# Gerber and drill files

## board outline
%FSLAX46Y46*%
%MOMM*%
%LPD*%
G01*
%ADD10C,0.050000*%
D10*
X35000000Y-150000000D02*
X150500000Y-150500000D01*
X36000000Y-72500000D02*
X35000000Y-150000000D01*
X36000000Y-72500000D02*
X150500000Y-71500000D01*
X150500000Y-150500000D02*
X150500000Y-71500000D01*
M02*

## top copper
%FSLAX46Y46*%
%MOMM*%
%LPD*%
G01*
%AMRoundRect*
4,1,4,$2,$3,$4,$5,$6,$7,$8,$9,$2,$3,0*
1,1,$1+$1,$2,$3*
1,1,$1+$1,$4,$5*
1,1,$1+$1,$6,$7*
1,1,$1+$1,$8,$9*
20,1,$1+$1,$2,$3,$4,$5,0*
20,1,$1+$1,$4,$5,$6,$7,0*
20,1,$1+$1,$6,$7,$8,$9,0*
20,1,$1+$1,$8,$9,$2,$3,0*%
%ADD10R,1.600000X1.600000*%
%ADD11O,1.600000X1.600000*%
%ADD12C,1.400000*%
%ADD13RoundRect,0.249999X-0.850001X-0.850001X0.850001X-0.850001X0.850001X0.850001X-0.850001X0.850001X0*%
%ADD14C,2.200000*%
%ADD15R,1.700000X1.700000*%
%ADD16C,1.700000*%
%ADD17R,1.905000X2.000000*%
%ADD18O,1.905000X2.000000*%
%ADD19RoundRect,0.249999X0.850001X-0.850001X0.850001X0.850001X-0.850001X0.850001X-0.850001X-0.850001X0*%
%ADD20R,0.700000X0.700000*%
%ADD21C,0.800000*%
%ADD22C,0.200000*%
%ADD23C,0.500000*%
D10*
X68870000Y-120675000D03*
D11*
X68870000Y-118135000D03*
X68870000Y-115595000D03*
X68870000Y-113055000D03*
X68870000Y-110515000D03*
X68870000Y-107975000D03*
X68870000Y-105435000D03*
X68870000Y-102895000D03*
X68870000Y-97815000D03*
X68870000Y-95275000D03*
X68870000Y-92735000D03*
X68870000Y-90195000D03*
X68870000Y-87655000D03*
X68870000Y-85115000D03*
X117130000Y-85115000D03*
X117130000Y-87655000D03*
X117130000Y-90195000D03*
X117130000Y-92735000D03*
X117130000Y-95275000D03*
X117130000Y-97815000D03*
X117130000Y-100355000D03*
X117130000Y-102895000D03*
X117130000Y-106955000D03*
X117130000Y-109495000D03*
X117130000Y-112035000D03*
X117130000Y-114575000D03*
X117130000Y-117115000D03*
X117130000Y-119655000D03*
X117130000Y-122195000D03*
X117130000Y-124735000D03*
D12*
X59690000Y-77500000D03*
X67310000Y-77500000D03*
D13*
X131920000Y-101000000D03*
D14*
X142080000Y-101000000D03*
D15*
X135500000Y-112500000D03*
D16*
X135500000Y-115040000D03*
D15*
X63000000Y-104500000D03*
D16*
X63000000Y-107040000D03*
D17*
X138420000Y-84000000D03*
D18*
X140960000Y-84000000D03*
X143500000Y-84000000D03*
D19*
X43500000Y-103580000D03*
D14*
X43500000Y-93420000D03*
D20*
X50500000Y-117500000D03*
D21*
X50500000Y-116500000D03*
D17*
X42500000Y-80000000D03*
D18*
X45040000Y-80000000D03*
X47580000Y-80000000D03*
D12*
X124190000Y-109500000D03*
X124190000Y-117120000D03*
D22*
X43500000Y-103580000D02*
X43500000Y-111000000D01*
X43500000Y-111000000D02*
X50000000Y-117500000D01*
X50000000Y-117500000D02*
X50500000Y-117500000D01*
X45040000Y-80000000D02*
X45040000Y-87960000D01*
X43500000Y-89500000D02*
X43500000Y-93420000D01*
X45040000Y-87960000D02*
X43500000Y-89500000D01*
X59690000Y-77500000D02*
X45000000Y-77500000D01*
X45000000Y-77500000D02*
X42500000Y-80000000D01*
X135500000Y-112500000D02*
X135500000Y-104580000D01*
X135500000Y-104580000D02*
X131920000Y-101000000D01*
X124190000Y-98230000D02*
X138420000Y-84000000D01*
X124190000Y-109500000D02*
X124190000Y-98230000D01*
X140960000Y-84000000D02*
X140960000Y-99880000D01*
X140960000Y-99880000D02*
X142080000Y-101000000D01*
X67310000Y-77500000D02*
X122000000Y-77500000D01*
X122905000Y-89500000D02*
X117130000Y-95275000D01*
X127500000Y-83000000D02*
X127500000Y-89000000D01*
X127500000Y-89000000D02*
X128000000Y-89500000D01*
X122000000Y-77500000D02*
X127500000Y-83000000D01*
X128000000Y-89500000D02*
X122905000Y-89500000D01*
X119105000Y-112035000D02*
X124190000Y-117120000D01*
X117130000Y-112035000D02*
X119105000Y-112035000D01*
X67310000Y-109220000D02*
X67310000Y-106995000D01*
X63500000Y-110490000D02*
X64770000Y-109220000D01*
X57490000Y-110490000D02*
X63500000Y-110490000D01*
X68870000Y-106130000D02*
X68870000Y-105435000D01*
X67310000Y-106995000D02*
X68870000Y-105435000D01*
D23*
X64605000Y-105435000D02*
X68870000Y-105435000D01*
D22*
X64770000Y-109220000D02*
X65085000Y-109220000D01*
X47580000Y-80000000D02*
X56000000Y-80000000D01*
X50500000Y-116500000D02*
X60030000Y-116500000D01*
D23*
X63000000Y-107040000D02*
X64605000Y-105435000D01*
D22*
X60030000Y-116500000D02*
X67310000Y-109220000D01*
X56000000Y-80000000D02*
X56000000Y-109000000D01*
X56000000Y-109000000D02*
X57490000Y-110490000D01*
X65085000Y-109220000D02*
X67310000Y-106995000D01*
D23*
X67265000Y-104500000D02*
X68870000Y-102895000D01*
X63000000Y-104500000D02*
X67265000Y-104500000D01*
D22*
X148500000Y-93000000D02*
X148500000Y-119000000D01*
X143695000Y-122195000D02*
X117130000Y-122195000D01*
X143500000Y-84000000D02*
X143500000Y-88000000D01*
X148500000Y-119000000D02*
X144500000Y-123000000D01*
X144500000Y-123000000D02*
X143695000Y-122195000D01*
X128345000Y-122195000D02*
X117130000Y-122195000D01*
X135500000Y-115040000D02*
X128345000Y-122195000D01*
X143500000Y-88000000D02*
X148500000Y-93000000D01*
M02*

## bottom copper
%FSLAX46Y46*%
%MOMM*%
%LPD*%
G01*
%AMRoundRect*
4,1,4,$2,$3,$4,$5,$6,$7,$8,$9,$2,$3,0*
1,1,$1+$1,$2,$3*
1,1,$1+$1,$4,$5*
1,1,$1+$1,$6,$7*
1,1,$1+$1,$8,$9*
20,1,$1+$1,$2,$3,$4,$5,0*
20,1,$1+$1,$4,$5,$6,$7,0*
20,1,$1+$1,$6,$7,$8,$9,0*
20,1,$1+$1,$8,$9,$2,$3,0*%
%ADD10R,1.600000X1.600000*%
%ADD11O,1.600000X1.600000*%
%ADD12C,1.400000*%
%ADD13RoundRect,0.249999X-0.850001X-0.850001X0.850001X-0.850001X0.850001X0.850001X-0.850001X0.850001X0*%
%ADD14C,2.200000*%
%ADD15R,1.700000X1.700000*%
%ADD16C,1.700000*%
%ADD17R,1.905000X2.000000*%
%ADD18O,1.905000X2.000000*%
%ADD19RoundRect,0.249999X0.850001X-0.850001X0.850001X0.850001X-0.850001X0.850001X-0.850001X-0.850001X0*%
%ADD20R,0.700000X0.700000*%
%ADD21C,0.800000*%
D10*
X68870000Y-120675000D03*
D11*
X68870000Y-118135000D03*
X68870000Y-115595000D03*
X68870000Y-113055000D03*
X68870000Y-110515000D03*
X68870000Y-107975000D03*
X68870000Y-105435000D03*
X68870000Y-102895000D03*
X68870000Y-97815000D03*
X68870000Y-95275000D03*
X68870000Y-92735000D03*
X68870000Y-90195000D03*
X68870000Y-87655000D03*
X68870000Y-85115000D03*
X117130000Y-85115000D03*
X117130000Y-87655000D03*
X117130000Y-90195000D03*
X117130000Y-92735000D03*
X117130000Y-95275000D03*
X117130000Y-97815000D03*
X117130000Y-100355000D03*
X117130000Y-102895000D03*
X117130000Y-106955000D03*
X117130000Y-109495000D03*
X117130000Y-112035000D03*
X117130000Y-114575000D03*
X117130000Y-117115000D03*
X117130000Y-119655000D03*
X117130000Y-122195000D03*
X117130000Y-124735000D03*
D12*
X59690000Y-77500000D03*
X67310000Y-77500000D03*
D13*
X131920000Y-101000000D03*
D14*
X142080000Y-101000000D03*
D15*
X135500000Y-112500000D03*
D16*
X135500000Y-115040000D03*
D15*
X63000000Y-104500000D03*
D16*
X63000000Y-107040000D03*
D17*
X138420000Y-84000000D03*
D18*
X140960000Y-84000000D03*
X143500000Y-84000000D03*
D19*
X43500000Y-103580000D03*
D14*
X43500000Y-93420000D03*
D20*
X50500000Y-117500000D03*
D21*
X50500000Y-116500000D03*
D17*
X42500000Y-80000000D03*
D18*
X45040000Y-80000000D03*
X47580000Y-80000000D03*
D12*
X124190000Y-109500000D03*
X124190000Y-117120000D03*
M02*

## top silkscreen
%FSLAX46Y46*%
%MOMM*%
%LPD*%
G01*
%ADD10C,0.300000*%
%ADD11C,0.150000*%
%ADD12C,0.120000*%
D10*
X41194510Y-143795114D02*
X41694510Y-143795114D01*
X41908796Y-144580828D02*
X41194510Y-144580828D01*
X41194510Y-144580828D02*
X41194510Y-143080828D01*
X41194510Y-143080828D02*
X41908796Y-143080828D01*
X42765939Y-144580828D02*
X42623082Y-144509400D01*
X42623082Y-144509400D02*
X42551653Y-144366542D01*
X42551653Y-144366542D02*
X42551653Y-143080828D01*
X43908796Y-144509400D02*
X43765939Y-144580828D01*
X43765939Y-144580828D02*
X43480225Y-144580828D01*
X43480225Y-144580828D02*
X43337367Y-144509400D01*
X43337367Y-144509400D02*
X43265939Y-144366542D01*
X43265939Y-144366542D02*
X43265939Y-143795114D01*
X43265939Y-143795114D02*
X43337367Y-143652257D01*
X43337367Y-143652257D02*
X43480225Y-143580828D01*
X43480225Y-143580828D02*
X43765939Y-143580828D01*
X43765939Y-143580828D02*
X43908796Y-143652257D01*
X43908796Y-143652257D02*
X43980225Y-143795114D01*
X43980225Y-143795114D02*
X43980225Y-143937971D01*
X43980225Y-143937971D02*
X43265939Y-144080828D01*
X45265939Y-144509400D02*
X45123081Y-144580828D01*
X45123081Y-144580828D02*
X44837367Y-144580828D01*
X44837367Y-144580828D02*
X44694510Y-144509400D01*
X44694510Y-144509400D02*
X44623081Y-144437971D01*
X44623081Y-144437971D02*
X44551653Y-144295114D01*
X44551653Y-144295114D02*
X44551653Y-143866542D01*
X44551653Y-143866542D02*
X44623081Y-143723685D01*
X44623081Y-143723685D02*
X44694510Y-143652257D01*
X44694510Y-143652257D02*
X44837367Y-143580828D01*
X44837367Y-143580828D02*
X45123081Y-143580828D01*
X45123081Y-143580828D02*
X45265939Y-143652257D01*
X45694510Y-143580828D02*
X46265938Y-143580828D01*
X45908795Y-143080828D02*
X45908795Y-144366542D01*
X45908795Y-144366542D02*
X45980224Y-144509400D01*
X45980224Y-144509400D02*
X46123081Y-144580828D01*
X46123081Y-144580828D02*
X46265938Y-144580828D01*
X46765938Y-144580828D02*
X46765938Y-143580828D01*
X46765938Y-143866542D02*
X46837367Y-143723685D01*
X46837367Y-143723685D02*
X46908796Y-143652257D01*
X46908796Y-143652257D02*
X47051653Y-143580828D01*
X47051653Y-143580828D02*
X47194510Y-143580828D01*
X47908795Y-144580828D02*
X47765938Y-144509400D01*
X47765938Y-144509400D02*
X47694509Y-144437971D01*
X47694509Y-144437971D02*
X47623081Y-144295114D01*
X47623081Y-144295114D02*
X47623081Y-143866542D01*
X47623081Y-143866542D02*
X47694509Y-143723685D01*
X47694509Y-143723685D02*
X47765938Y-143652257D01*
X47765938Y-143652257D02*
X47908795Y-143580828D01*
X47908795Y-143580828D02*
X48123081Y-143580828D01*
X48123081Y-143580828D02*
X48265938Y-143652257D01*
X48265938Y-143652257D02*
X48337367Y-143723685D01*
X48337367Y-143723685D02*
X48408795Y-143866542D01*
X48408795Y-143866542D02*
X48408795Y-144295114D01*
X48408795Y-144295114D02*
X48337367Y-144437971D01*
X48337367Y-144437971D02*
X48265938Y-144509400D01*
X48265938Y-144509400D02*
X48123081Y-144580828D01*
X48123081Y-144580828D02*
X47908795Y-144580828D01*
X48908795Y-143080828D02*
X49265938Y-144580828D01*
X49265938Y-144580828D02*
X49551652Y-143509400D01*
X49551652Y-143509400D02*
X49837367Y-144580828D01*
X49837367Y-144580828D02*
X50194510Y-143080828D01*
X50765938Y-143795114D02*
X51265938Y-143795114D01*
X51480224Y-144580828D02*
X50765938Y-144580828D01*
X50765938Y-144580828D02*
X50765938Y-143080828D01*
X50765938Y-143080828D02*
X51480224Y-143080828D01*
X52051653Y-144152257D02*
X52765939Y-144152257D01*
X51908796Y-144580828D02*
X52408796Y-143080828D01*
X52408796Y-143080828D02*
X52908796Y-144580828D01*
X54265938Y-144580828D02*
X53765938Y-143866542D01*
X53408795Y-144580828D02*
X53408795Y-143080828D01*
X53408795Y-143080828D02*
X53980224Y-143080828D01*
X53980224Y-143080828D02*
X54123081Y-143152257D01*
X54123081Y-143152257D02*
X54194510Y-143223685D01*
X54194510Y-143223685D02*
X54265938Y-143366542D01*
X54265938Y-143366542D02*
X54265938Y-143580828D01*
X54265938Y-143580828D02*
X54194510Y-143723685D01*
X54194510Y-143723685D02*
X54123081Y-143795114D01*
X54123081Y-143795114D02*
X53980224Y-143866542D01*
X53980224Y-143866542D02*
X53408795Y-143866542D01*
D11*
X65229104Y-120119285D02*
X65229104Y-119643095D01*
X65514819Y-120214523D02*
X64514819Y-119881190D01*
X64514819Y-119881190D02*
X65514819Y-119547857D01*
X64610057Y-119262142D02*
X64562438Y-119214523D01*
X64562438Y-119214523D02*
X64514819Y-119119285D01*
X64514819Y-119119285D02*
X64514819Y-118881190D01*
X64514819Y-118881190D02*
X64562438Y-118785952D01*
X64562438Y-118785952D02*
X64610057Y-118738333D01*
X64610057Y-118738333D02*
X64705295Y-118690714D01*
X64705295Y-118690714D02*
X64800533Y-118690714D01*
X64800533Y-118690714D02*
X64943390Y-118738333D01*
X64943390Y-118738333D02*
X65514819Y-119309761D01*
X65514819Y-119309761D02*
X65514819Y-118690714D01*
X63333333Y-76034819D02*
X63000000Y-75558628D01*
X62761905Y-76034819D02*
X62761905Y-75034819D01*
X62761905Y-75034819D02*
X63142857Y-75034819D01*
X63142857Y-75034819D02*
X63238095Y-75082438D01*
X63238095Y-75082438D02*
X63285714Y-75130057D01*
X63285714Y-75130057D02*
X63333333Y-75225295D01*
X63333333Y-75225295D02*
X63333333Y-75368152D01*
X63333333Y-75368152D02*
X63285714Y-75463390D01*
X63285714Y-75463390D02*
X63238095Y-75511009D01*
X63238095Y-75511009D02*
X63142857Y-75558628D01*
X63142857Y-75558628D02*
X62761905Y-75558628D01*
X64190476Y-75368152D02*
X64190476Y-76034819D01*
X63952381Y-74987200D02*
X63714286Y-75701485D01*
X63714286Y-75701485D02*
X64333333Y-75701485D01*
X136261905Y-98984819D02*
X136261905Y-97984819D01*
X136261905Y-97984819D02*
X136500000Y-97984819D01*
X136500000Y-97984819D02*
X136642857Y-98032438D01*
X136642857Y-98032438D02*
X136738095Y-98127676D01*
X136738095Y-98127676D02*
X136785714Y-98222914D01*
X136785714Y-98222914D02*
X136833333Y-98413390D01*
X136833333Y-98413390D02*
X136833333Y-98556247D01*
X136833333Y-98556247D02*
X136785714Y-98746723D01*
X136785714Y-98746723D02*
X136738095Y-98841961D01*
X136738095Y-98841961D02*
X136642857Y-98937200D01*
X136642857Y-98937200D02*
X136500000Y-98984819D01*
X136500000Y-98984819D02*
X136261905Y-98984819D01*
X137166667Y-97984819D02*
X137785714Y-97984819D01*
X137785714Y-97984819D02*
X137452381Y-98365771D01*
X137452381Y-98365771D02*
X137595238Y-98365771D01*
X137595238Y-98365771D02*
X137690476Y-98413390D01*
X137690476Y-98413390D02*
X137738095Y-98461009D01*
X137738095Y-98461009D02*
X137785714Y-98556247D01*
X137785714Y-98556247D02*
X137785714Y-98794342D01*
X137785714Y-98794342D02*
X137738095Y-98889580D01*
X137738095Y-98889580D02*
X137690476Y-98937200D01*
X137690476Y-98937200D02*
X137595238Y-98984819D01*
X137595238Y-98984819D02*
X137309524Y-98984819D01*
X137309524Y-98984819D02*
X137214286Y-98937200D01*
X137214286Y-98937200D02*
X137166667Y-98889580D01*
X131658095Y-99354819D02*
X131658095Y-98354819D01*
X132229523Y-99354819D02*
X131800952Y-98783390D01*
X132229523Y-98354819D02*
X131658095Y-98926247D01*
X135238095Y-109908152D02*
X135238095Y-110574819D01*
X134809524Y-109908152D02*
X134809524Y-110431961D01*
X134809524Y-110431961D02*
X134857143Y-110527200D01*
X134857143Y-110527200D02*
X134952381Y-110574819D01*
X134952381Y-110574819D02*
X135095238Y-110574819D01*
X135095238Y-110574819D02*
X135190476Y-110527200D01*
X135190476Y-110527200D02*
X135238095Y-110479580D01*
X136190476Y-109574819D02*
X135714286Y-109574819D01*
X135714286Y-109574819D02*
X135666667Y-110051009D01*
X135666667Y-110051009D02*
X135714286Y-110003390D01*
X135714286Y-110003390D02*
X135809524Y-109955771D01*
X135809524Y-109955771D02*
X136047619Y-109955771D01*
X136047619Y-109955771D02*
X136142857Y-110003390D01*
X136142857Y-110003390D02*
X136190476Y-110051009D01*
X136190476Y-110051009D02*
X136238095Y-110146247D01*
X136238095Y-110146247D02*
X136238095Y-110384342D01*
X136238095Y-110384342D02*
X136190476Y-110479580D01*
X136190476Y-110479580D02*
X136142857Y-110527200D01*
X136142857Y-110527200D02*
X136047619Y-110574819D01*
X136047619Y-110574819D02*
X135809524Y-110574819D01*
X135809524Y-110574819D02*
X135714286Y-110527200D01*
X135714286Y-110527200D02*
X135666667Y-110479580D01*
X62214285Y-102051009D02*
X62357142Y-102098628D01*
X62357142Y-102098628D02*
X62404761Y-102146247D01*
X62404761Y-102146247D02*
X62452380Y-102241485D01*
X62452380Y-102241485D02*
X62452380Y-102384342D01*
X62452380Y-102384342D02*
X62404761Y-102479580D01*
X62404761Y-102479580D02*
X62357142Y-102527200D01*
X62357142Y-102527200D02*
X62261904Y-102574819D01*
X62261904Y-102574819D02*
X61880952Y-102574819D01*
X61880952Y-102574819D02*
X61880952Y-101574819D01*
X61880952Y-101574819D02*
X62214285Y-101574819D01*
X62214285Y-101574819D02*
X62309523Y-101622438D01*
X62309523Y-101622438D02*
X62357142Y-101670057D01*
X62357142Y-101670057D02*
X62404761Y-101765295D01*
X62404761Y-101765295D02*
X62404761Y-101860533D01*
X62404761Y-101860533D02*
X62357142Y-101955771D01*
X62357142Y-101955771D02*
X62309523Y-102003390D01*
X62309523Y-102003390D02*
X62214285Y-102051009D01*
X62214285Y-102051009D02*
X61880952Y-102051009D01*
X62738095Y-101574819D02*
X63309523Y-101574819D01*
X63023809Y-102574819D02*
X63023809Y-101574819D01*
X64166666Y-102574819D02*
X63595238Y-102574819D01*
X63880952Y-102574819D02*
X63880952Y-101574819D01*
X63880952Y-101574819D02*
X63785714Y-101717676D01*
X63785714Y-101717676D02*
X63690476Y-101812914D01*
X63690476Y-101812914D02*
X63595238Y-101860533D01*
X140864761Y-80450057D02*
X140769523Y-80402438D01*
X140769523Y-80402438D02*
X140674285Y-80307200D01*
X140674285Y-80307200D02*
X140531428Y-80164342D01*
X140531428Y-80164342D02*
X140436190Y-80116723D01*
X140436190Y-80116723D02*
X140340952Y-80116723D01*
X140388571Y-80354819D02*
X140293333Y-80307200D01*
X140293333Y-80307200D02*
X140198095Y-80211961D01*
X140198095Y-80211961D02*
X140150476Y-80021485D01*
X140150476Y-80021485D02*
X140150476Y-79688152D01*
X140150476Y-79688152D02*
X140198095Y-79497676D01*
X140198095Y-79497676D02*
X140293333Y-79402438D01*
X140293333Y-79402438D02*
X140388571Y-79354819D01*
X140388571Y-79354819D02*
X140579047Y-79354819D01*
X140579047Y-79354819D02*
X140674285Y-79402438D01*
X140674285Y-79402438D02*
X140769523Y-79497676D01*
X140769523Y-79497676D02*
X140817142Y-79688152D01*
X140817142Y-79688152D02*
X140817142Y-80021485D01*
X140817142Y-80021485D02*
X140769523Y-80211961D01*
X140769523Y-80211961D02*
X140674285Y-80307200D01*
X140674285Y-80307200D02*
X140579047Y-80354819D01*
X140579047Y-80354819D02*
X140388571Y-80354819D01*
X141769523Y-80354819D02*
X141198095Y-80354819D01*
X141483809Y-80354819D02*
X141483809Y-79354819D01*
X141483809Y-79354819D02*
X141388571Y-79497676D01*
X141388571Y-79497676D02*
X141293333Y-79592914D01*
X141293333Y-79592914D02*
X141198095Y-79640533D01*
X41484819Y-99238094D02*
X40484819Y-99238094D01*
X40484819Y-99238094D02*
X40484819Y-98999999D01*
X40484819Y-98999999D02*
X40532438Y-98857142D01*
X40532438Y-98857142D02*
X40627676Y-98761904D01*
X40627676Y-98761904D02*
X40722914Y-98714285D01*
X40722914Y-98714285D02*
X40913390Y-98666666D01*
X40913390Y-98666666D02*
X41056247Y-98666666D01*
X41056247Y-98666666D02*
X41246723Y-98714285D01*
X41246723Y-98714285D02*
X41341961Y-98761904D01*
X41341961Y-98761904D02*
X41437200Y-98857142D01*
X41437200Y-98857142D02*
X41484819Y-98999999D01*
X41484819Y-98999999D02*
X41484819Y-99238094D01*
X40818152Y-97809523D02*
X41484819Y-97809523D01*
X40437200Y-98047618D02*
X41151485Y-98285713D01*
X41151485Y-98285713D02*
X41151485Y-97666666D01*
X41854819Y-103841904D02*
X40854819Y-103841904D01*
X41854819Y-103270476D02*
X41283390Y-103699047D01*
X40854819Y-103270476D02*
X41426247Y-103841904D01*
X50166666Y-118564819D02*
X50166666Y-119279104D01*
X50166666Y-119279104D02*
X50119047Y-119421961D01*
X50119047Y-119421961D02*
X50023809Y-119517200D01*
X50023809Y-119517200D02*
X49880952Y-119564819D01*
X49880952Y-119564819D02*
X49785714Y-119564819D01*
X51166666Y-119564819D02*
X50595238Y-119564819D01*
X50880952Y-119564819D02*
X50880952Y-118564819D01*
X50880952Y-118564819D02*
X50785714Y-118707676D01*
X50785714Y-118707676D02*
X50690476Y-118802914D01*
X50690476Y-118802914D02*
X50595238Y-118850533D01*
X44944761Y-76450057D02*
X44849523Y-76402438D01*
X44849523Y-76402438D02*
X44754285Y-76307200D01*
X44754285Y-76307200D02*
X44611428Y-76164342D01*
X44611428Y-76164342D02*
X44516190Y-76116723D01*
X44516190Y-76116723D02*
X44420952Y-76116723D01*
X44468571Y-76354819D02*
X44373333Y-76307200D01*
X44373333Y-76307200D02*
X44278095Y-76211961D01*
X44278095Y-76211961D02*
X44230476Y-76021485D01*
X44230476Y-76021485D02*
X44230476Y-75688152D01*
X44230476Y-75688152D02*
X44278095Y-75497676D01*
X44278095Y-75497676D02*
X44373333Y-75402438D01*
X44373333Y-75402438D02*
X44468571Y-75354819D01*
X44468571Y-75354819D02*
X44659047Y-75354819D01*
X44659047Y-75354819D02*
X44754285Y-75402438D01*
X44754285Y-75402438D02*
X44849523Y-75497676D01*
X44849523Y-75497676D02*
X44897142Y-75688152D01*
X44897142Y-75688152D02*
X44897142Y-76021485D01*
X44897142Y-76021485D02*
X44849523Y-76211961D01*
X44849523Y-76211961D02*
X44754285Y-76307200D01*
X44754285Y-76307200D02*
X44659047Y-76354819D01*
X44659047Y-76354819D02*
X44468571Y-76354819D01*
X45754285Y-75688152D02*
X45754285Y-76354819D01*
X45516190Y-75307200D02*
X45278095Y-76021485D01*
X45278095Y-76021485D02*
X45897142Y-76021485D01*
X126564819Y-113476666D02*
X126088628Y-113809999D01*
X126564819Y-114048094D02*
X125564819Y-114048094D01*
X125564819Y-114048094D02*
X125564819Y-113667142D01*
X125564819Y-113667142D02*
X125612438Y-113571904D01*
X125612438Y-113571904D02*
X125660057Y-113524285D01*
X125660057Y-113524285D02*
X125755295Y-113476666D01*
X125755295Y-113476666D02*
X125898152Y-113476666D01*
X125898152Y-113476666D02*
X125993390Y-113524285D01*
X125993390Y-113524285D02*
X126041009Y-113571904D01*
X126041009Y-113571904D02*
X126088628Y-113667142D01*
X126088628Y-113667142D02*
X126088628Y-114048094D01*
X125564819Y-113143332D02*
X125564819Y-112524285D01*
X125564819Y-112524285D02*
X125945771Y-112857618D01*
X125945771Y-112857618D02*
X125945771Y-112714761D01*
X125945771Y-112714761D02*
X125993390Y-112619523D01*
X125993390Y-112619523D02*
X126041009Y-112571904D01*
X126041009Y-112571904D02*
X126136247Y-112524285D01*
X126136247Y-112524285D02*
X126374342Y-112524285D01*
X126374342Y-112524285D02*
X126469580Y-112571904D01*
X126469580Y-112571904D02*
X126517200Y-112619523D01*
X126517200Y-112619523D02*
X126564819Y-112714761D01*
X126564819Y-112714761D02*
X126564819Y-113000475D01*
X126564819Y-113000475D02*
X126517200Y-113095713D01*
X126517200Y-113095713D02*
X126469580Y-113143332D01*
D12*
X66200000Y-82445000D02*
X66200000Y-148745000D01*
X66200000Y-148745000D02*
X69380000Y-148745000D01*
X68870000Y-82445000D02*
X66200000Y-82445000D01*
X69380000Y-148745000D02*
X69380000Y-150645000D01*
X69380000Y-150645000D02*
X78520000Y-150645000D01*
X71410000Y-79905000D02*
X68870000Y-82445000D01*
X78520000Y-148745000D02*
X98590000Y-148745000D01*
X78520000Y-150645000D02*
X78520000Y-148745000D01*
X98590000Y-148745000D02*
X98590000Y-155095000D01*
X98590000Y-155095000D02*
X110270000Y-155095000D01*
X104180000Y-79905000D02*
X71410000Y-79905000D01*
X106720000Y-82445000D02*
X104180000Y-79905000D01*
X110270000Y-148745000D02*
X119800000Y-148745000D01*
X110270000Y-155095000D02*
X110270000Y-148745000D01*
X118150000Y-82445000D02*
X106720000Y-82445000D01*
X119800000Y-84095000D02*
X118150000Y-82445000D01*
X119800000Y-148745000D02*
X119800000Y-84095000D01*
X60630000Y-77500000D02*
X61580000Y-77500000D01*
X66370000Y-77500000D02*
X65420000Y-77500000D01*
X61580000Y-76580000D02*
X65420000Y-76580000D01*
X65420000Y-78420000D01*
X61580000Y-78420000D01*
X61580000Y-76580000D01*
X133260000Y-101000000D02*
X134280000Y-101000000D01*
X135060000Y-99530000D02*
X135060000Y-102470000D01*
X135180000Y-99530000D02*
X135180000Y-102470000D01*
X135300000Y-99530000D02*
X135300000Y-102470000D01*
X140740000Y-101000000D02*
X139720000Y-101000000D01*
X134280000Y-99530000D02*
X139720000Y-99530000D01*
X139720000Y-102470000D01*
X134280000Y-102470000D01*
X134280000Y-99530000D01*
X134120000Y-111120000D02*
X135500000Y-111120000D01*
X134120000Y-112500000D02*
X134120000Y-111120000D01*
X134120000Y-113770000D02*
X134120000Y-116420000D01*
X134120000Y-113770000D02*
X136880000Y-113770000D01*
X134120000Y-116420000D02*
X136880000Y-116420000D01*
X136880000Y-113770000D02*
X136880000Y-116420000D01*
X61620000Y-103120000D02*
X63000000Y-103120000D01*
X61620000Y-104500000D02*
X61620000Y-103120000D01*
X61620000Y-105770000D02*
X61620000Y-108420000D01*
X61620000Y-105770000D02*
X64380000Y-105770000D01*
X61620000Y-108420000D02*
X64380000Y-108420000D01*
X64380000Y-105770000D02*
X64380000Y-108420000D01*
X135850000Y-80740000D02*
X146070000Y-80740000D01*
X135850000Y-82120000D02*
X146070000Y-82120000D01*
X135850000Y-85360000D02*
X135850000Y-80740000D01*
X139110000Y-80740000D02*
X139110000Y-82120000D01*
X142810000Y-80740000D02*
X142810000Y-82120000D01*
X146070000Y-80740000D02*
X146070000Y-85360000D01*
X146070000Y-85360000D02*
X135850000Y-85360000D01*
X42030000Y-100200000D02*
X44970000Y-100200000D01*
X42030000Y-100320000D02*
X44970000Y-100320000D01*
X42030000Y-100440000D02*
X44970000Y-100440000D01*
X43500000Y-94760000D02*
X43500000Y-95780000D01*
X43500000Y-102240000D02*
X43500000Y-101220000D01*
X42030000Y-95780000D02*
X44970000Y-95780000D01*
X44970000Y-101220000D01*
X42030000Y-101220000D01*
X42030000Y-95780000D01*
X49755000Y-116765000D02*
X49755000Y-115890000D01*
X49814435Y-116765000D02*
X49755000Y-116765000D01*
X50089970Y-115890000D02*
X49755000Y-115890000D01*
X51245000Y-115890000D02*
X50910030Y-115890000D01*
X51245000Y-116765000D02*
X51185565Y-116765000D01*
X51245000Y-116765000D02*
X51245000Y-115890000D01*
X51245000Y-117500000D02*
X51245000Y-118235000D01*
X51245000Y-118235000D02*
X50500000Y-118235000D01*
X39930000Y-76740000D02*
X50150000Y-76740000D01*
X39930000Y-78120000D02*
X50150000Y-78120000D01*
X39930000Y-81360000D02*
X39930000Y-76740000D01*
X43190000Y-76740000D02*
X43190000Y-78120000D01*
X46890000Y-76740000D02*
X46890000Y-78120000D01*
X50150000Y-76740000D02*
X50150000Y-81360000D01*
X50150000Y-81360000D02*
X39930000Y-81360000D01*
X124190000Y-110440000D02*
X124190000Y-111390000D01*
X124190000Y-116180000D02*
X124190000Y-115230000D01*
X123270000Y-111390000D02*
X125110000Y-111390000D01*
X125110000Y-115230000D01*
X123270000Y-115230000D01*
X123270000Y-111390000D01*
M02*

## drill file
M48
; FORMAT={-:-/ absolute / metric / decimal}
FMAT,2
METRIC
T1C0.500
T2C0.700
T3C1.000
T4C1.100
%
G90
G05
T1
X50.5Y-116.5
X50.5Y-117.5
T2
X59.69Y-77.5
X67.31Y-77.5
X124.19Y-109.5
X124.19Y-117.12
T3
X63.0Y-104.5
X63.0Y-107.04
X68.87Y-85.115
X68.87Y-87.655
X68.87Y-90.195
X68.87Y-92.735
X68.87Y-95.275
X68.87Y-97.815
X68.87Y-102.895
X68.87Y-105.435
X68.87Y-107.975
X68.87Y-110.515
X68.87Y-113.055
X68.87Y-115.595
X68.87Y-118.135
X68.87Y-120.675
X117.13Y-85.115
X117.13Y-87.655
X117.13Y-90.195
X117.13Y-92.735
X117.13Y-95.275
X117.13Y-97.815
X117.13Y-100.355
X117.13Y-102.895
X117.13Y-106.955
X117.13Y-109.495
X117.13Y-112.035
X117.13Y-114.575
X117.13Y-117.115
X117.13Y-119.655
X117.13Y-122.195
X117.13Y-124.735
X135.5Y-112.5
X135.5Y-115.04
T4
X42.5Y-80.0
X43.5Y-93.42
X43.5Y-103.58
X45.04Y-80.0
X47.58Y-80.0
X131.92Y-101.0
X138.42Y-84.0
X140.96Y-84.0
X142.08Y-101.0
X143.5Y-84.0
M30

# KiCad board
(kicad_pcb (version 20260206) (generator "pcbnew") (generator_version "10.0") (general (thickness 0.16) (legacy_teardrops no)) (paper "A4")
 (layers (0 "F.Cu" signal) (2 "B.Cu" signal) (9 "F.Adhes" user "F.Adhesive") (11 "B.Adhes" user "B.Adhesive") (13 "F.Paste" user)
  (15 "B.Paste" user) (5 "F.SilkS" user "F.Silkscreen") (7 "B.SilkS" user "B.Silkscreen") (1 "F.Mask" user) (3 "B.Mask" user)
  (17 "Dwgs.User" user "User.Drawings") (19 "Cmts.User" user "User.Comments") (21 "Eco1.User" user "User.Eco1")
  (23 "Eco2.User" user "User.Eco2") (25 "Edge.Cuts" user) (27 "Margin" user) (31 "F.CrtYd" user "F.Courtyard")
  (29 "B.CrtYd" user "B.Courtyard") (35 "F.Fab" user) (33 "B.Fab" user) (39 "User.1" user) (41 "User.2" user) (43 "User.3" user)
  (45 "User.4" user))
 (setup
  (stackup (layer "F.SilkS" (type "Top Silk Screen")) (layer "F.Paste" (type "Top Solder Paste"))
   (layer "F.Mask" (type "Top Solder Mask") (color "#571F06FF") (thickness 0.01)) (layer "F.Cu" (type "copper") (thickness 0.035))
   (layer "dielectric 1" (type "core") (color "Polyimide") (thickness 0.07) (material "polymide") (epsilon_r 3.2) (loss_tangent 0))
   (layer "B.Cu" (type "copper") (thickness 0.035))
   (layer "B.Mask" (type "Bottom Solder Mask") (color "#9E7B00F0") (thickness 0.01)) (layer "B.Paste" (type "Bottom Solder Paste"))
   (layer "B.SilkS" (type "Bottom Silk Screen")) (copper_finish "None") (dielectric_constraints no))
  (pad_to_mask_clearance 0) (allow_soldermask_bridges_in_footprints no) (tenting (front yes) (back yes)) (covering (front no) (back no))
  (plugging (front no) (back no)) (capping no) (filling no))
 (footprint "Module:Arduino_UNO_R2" (layer "F.Cu") (at 68.87 120.675 90)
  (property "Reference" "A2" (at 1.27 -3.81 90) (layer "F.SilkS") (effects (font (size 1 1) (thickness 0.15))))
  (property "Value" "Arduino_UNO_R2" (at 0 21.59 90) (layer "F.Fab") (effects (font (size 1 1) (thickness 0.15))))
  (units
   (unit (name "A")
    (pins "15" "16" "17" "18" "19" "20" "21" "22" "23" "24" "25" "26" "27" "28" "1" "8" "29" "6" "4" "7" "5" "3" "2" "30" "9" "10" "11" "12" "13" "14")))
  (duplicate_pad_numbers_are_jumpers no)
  (fp_line (start 38.23 -2.67) (end -28.07 -2.67) (stroke (width 0.12) (type solid)) (layer "F.SilkS"))
  (fp_line (start -28.07 -2.67) (end -28.07 0.51) (stroke (width 0.12) (type solid)) (layer "F.SilkS"))
  (fp_line (start 38.23 0) (end 38.23 -2.67) (stroke (width 0.12) (type solid)) (layer "F.SilkS"))
  (fp_line (start -28.07 0.51) (end -29.97 0.51) (stroke (width 0.12) (type solid)) (layer "F.SilkS"))
  (fp_line (start -29.97 0.51) (end -29.97 9.65) (stroke (width 0.12) (type solid)) (layer "F.SilkS"))
  (fp_line (start 40.77 2.54) (end 38.23 0) (stroke (width 0.12) (type solid)) (layer "F.SilkS"))
  (fp_line (start -28.07 9.65) (end -28.07 29.72) (stroke (width 0.12) (type solid)) (layer "F.SilkS"))
  (fp_line (start -29.97 9.65) (end -28.07 9.65) (stroke (width 0.12) (type solid)) (layer "F.SilkS"))
  (fp_line (start -28.07 29.72) (end -34.42 29.72) (stroke (width 0.12) (type solid)) (layer "F.SilkS"))
  (fp_line (start -34.42 29.72) (end -34.42 41.4) (stroke (width 0.12) (type solid)) (layer "F.SilkS"))
  (fp_line (start 40.77 35.31) (end 40.77 2.54) (stroke (width 0.12) (type solid)) (layer "F.SilkS"))
  (fp_line (start 38.23 37.85) (end 40.77 35.31) (stroke (width 0.12) (type solid)) (layer "F.SilkS"))
  (fp_line (start -28.07 41.4) (end -28.07 50.93) (stroke (width 0.12) (type solid)) (layer "F.SilkS"))
  (fp_line (start -34.42 41.4) (end -28.07 41.4) (stroke (width 0.12) (type solid)) (layer "F.SilkS"))
  (fp_line (start 38.23 49.28) (end 38.23 37.85) (stroke (width 0.12) (type solid)) (layer "F.SilkS"))
  (fp_line (start 36.58 50.93) (end 38.23 49.28) (stroke (width 0.12) (type solid)) (layer "F.SilkS"))
  (fp_line (start -28.07 50.93) (end 36.58 50.93) (stroke (width 0.12) (type solid)) (layer "F.SilkS"))
  (pad "1" thru_hole rect (at 0 0 180) (size 1.6 1.6) (drill 1) (layers "*.Cu" "*.Mask") (remove_unused_layers no)
   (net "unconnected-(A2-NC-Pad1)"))
  (pad "2" thru_hole oval (at 2.54 0 180) (size 1.6 1.6) (drill 1) (layers "*.Cu" "*.Mask") (remove_unused_layers no)
   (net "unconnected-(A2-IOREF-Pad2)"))
  (pad "3" thru_hole oval (at 5.08 0 180) (size 1.6 1.6) (drill 1) (layers "*.Cu" "*.Mask") (remove_unused_layers no)
   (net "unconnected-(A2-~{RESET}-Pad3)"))
  (pad "4" thru_hole oval (at 7.62 0 180) (size 1.6 1.6) (drill 1) (layers "*.Cu" "*.Mask") (remove_unused_layers no)
   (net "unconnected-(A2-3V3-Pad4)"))
  (pad "5" thru_hole oval (at 10.16 0 180) (size 1.6 1.6) (drill 1) (layers "*.Cu" "*.Mask") (remove_unused_layers no)
   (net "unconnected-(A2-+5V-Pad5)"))
  (pad "6" thru_hole oval (at 12.7 0 180) (size 1.6 1.6) (drill 1) (layers "*.Cu" "*.Mask") (remove_unused_layers no)
   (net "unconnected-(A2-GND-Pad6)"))
  (pad "7" thru_hole oval (at 15.24 0 180) (size 1.6 1.6) (drill 1) (layers "*.Cu" "*.Mask") (remove_unused_layers no) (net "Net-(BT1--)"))
  (pad "8" thru_hole oval (at 17.78 0 180) (size 1.6 1.6) (drill 1) (layers "*.Cu" "*.Mask") (remove_unused_layers no) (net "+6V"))
  (pad "9" thru_hole oval (at 22.86 0 180) (size 1.6 1.6) (drill 1) (layers "*.Cu" "*.Mask") (remove_unused_layers no)
   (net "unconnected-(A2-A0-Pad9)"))
  (pad "10" thru_hole oval (at 25.4 0 180) (size 1.6 1.6) (drill 1) (layers "*.Cu" "*.Mask") (remove_unused_layers no)
   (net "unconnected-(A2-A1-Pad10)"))
  (pad "11" thru_hole oval (at 27.94 0 180) (size 1.6 1.6) (drill 1) (layers "*.Cu" "*.Mask") (remove_unused_layers no)
   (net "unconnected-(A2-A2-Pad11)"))
  (pad "12" thru_hole oval (at 30.48 0 180) (size 1.6 1.6) (drill 1) (layers "*.Cu" "*.Mask") (remove_unused_layers no)
   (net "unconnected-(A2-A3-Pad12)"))
  (pad "13" thru_hole oval (at 33.02 0 180) (size 1.6 1.6) (drill 1) (layers "*.Cu" "*.Mask") (remove_unused_layers no)
   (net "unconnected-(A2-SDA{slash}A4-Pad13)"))
  (pad "14" thru_hole oval (at 35.56 0 180) (size 1.6 1.6) (drill 1) (layers "*.Cu" "*.Mask") (remove_unused_layers no)
   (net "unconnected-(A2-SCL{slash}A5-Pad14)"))
  (pad "15" thru_hole oval (at 35.56 48.26 180) (size 1.6 1.6) (drill 1) (layers "*.Cu" "*.Mask") (remove_unused_layers no)
   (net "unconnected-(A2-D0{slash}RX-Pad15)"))
  (pad "16" thru_hole oval (at 33.02 48.26 180) (size 1.6 1.6) (drill 1) (layers "*.Cu" "*.Mask") (remove_unused_layers no)
   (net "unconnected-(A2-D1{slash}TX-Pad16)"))
  (pad "17" thru_hole oval (at 30.48 48.26 180) (size 1.6 1.6) (drill 1) (layers "*.Cu" "*.Mask") (remove_unused_layers no)
   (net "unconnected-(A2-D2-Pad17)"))
  (pad "18" thru_hole oval (at 27.94 48.26 180) (size 1.6 1.6) (drill 1) (layers "*.Cu" "*.Mask") (remove_unused_layers no)
   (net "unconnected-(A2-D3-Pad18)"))
  (pad "19" thru_hole oval (at 25.4 48.26 180) (size 1.6 1.6) (drill 1) (layers "*.Cu" "*.Mask") (remove_unused_layers no)
   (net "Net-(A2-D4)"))
  (pad "20" thru_hole oval (at 22.86 48.26 180) (size 1.6 1.6) (drill 1) (layers "*.Cu" "*.Mask") (remove_unused_layers no)
   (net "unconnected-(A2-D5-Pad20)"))
  (pad "21" thru_hole oval (at 20.32 48.26 180) (size 1.6 1.6) (drill 1) (layers "*.Cu" "*.Mask") (remove_unused_layers no)
   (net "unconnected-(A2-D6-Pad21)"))
  (pad "22" thru_hole oval (at 17.78 48.26 180) (size 1.6 1.6) (drill 1) (layers "*.Cu" "*.Mask") (remove_unused_layers no)
   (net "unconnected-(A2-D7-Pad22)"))
  (pad "23" thru_hole oval (at 13.72 48.26 180) (size 1.6 1.6) (drill 1) (layers "*.Cu" "*.Mask") (remove_unused_layers no)
   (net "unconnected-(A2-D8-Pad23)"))
  (pad "24" thru_hole oval (at 11.18 48.26 180) (size 1.6 1.6) (drill 1) (layers "*.Cu" "*.Mask") (remove_unused_layers no)
   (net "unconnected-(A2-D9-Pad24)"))
  (pad "25" thru_hole oval (at 8.64 48.26 180) (size 1.6 1.6) (drill 1) (layers "*.Cu" "*.Mask") (remove_unused_layers no)
   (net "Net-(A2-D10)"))
  (pad "26" thru_hole oval (at 6.1 48.26 180) (size 1.6 1.6) (drill 1) (layers "*.Cu" "*.Mask") (remove_unused_layers no)
   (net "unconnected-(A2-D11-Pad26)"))
  (pad "27" thru_hole oval (at 3.56 48.26 180) (size 1.6 1.6) (drill 1) (layers "*.Cu" "*.Mask") (remove_unused_layers no)
   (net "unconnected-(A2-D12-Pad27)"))
  (pad "28" thru_hole oval (at 1.02 48.26 180) (size 1.6 1.6) (drill 1) (layers "*.Cu" "*.Mask") (remove_unused_layers no)
   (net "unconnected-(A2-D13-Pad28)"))
  (pad "29" thru_hole oval (at -1.52 48.26 180) (size 1.6 1.6) (drill 1) (layers "*.Cu" "*.Mask") (remove_unused_layers no)
   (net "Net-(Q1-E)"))
  (pad "30" thru_hole oval (at -4.06 48.26 180) (size 1.6 1.6) (drill 1) (layers "*.Cu" "*.Mask") (remove_unused_layers no)
   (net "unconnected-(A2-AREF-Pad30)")))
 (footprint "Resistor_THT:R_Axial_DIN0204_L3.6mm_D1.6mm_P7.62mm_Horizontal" (layer "F.Cu") (at 59.69 77.5)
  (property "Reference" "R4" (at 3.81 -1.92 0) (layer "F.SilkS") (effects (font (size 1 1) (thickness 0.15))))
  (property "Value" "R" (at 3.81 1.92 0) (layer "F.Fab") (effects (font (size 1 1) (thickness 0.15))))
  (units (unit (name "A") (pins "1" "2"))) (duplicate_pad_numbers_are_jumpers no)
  (fp_line (start 0.94 0) (end 1.89 0) (stroke (width 0.12) (type solid)) (layer "F.SilkS"))
  (fp_line (start 6.68 0) (end 5.73 0) (stroke (width 0.12) (type solid)) (layer "F.SilkS"))
  (fp_rect (start 1.89 -0.92) (end 5.73 0.92) (stroke (width 0.12) (type solid)) (fill no) (layer "F.SilkS"))
  (pad "1" thru_hole circle (at 0 0) (size 1.4 1.4) (drill 0.7) (layers "*.Cu" "*.Mask") (remove_unused_layers no) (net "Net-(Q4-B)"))
  (pad "2" thru_hole circle (at 7.62 0) (size 1.4 1.4) (drill 0.7) (layers "*.Cu" "*.Mask") (remove_unused_layers no) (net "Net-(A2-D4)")))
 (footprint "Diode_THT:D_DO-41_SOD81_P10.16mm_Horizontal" (layer "F.Cu") (at 131.92 101)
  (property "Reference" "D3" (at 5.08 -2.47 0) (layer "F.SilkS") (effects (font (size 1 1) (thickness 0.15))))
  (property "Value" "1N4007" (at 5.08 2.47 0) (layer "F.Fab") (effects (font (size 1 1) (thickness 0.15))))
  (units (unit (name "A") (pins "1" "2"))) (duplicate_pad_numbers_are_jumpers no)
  (fp_line (start 1.34 0) (end 2.36 0) (stroke (width 0.12) (type solid)) (layer "F.SilkS"))
  (fp_line (start 3.14 -1.47) (end 3.14 1.47) (stroke (width 0.12) (type solid)) (layer "F.SilkS"))
  (fp_line (start 3.26 -1.47) (end 3.26 1.47) (stroke (width 0.12) (type solid)) (layer "F.SilkS"))
  (fp_line (start 3.38 -1.47) (end 3.38 1.47) (stroke (width 0.12) (type solid)) (layer "F.SilkS"))
  (fp_line (start 8.82 0) (end 7.8 0) (stroke (width 0.12) (type solid)) (layer "F.SilkS"))
  (fp_rect (start 2.36 -1.47) (end 7.8 1.47) (stroke (width 0.12) (type solid)) (fill no) (layer "F.SilkS"))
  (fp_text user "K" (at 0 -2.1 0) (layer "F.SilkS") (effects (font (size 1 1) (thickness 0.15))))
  (pad "1" thru_hole roundrect (at 0 0) (size 2.2 2.2) (drill 1.1) (layers "*.Cu" "*.Mask") (remove_unused_layers no)
   (roundrect_rratio 0.113636) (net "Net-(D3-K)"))
  (pad "2" thru_hole circle (at 10.16 0) (size 2.2 2.2) (drill 1.1) (layers "*.Cu" "*.Mask") (remove_unused_layers no) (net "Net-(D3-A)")))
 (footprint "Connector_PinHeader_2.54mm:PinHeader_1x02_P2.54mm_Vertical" (layer "F.Cu") (at 135.5 112.5)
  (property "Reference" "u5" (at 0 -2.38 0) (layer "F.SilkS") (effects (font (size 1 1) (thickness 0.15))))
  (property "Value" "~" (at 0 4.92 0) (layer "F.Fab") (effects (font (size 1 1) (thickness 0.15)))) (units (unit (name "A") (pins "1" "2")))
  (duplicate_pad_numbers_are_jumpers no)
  (fp_line (start -1.38 -1.38) (end 0 -1.38) (stroke (width 0.12) (type solid)) (layer "F.SilkS"))
  (fp_line (start -1.38 0) (end -1.38 -1.38) (stroke (width 0.12) (type solid)) (layer "F.SilkS"))
  (fp_line (start -1.38 1.27) (end -1.38 3.92) (stroke (width 0.12) (type solid)) (layer "F.SilkS"))
  (fp_line (start -1.38 1.27) (end 1.38 1.27) (stroke (width 0.12) (type solid)) (layer "F.SilkS"))
  (fp_line (start -1.38 3.92) (end 1.38 3.92) (stroke (width 0.12) (type solid)) (layer "F.SilkS"))
  (fp_line (start 1.38 1.27) (end 1.38 3.92) (stroke (width 0.12) (type solid)) (layer "F.SilkS"))
  (pad "1" thru_hole rect (at 0 0) (size 1.7 1.7) (drill 1) (layers "*.Cu" "*.Mask") (remove_unused_layers no) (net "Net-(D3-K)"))
  (pad "2" thru_hole circle (at 0 2.54) (size 1.7 1.7) (drill 1) (layers "*.Cu" "*.Mask") (remove_unused_layers no) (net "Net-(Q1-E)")))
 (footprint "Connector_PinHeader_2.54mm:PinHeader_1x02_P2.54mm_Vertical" (layer "F.Cu") (at 63 104.5)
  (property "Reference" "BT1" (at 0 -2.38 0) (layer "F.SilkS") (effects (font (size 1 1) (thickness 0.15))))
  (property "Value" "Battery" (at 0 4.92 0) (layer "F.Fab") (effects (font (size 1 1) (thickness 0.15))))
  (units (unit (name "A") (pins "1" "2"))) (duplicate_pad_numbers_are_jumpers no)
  (fp_line (start -1.38 -1.38) (end 0 -1.38) (stroke (width 0.12) (type solid)) (layer "F.SilkS"))
  (fp_line (start -1.38 0) (end -1.38 -1.38) (stroke (width 0.12) (type solid)) (layer "F.SilkS"))
  (fp_line (start -1.38 1.27) (end -1.38 3.92) (stroke (width 0.12) (type solid)) (layer "F.SilkS"))
  (fp_line (start -1.38 1.27) (end 1.38 1.27) (stroke (width 0.12) (type solid)) (layer "F.SilkS"))
  (fp_line (start -1.38 3.92) (end 1.38 3.92) (stroke (width 0.12) (type solid)) (layer "F.SilkS"))
  (fp_line (start 1.38 1.27) (end 1.38 3.92) (stroke (width 0.12) (type solid)) (layer "F.SilkS"))
  (pad "1" thru_hole rect (at 0 0) (size 1.7 1.7) (drill 1) (layers "*.Cu" "*.Mask") (remove_unused_layers no) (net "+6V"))
  (pad "2" thru_hole circle (at 0 2.54) (size 1.7 1.7) (drill 1) (layers "*.Cu" "*.Mask") (remove_unused_layers no) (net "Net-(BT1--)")))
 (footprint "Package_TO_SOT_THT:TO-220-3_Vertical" (layer "F.Cu") (at 138.42 84)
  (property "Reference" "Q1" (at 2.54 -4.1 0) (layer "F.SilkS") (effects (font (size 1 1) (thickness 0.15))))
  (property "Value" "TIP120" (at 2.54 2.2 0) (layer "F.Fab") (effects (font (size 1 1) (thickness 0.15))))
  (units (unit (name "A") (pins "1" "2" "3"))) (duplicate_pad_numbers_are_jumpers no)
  (fp_line (start -2.57 -3.26) (end 7.65 -3.26) (stroke (width 0.12) (type solid)) (layer "F.SilkS"))
  (fp_line (start -2.57 -1.88) (end 7.65 -1.88) (stroke (width 0.12) (type solid)) (layer "F.SilkS"))
  (fp_line (start -2.57 1.36) (end -2.57 -3.26) (stroke (width 0.12) (type solid)) (layer "F.SilkS"))
  (fp_line (start 0.69 -3.26) (end 0.69 -1.88) (stroke (width 0.12) (type solid)) (layer "F.SilkS"))
  (fp_line (start 4.39 -3.26) (end 4.39 -1.88) (stroke (width 0.12) (type solid)) (layer "F.SilkS"))
  (fp_line (start 7.65 -3.26) (end 7.65 1.36) (stroke (width 0.12) (type solid)) (layer "F.SilkS"))
  (fp_line (start 7.65 1.36) (end -2.57 1.36) (stroke (width 0.12) (type solid)) (layer "F.SilkS"))
  (pad "1" thru_hole rect (at 0 0) (size 1.905 2) (drill 1.1) (layers "*.Cu" "*.Mask") (remove_unused_layers no) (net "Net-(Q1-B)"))
  (pad "2" thru_hole oval (at 2.54 0) (size 1.905 2) (drill 1.1) (layers "*.Cu" "*.Mask") (remove_unused_layers no) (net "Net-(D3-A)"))
  (pad "3" thru_hole oval (at 5.08 0) (size 1.905 2) (drill 1.1) (layers "*.Cu" "*.Mask") (remove_unused_layers no) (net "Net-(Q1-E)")))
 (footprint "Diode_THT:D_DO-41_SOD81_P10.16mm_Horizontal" (layer "F.Cu") (at 43.5 103.58 90)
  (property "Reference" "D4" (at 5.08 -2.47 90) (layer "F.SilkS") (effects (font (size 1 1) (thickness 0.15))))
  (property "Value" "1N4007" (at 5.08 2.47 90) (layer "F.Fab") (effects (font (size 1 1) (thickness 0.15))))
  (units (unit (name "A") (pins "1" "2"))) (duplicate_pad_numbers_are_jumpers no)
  (fp_line (start 3.38 -1.47) (end 3.38 1.47) (stroke (width 0.12) (type solid)) (layer "F.SilkS"))
  (fp_line (start 3.26 -1.47) (end 3.26 1.47) (stroke (width 0.12) (type solid)) (layer "F.SilkS"))
  (fp_line (start 3.14 -1.47) (end 3.14 1.47) (stroke (width 0.12) (type solid)) (layer "F.SilkS"))
  (fp_line (start 8.82 0) (end 7.8 0) (stroke (width 0.12) (type solid)) (layer "F.SilkS"))
  (fp_line (start 1.34 0) (end 2.36 0) (stroke (width 0.12) (type solid)) (layer "F.SilkS"))
  (fp_rect (start 2.36 -1.47) (end 7.8 1.47) (stroke (width 0.12) (type solid)) (fill no) (layer "F.SilkS"))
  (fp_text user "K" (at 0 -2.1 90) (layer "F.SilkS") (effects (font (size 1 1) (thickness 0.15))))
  (pad "1" thru_hole roundrect (at 0 0 90) (size 2.2 2.2) (drill 1.1) (layers "*.Cu" "*.Mask") (remove_unused_layers no)
   (roundrect_rratio 0.113636) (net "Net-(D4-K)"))
  (pad "2" thru_hole circle (at 10.16 0 90) (size 2.2 2.2) (drill 1.1) (layers "*.Cu" "*.Mask") (remove_unused_layers no) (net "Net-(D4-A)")))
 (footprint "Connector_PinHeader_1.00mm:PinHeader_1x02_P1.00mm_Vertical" (layer "F.Cu") (at 50.5 117.5 180)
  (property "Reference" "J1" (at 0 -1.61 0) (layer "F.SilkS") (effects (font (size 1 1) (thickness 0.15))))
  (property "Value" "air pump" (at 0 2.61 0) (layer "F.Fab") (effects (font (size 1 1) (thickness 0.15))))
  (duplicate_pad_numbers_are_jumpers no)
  (fp_line (start 0.745 0.735) (end 0.745 1.61) (stroke (width 0.12) (type solid)) (layer "F.SilkS"))
  (fp_line (start 0.685565 0.735) (end 0.745 0.735) (stroke (width 0.12) (type solid)) (layer "F.SilkS"))
  (fp_line (start 0.41003 1.61) (end 0.745 1.61) (stroke (width 0.12) (type solid)) (layer "F.SilkS"))
  (fp_line (start -0.745 1.61) (end -0.41003 1.61) (stroke (width 0.12) (type solid)) (layer "F.SilkS"))
  (fp_line (start -0.745 0.735) (end -0.685565 0.735) (stroke (width 0.12) (type solid)) (layer "F.SilkS"))
  (fp_line (start -0.745 0.735) (end -0.745 1.61) (stroke (width 0.12) (type solid)) (layer "F.SilkS"))
  (fp_line (start -0.745 0) (end -0.745 -0.735) (stroke (width 0.12) (type solid)) (layer "F.SilkS"))
  (fp_line (start -0.745 -0.735) (end 0 -0.735) (stroke (width 0.12) (type solid)) (layer "F.SilkS"))
  (pad "1" thru_hole rect (at 0 0 180) (size 0.7 0.7) (drill 0.5) (layers "*.Cu" "*.Mask") (remove_unused_layers no) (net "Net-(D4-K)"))
  (pad "2" thru_hole circle (at 0 1 180) (size 0.8 0.8) (drill 0.5) (layers "*.Cu" "*.Mask") (remove_unused_layers no) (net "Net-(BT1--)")))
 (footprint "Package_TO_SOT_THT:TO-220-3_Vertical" (layer "F.Cu") (at 42.5 80)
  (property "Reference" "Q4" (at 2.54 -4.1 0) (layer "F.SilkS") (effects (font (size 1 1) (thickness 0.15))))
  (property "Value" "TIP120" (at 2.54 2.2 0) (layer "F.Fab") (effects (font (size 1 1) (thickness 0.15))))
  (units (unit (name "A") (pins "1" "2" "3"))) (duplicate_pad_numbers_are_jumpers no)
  (fp_line (start -2.57 -3.26) (end 7.65 -3.26) (stroke (width 0.12) (type solid)) (layer "F.SilkS"))
  (fp_line (start -2.57 -1.88) (end 7.65 -1.88) (stroke (width 0.12) (type solid)) (layer "F.SilkS"))
  (fp_line (start -2.57 1.36) (end -2.57 -3.26) (stroke (width 0.12) (type solid)) (layer "F.SilkS"))
  (fp_line (start 0.69 -3.26) (end 0.69 -1.88) (stroke (width 0.12) (type solid)) (layer "F.SilkS"))
  (fp_line (start 4.39 -3.26) (end 4.39 -1.88) (stroke (width 0.12) (type solid)) (layer "F.SilkS"))
  (fp_line (start 7.65 -3.26) (end 7.65 1.36) (stroke (width 0.12) (type solid)) (layer "F.SilkS"))
  (fp_line (start 7.65 1.36) (end -2.57 1.36) (stroke (width 0.12) (type solid)) (layer "F.SilkS"))
  (pad "1" thru_hole rect (at 0 0) (size 1.905 2) (drill 1.1) (layers "*.Cu" "*.Mask") (remove_unused_layers no) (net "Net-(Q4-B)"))
  (pad "2" thru_hole oval (at 2.54 0) (size 1.905 2) (drill 1.1) (layers "*.Cu" "*.Mask") (remove_unused_layers no) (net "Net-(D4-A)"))
  (pad "3" thru_hole oval (at 5.08 0) (size 1.905 2) (drill 1.1) (layers "*.Cu" "*.Mask") (remove_unused_layers no) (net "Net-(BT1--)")))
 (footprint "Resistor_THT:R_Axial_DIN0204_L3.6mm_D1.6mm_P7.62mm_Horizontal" (layer "F.Cu") (at 124.19 109.5 -90)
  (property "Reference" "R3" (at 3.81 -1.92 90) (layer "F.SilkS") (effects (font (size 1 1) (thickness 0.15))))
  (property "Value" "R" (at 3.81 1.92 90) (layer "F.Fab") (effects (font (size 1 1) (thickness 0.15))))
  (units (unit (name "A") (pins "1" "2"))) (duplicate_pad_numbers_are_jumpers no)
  (fp_line (start 0.94 0) (end 1.89 0) (stroke (width 0.12) (type solid)) (layer "F.SilkS"))
  (fp_line (start 6.68 0) (end 5.73 0) (stroke (width 0.12) (type solid)) (layer "F.SilkS"))
  (fp_rect (start 1.89 -0.92) (end 5.73 0.92) (stroke (width 0.12) (type solid)) (fill no) (layer "F.SilkS"))
  (pad "1" thru_hole circle (at 0 0 270) (size 1.4 1.4) (drill 0.7) (layers "*.Cu" "*.Mask") (remove_unused_layers no) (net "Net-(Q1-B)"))
  (pad "2" thru_hole circle (at 7.62 0 270) (size 1.4 1.4) (drill 0.7) (layers "*.Cu" "*.Mask") (remove_unused_layers no)
   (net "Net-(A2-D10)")))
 (gr_line (start 35 150) (end 150.5 150.5) (stroke (width 0.05) (type default)) (layer "Edge.Cuts"))
 (gr_line (start 36 72.5) (end 35 150) (stroke (width 0.05) (type default)) (layer "Edge.Cuts"))
 (gr_line (start 36 72.5) (end 150.5 71.5) (stroke (width 0.05) (type default)) (layer "Edge.Cuts"))
 (gr_line (start 150.5 150.5) (end 150.5 71.5) (stroke (width 0.05) (type default)) (layer "Edge.Cuts"))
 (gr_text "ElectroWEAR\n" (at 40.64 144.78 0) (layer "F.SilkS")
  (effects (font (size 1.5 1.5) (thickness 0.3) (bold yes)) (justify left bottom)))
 (segment (start 43.5 103.58) (end 43.5 111) (width 0.2) (layer "F.Cu") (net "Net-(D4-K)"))
 (segment (start 43.5 111) (end 50 117.5) (width 0.2) (layer "F.Cu") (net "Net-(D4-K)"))
 (segment (start 50 117.5) (end 50.5 117.5) (width 0.2) (layer "F.Cu") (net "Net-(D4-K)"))
 (segment (start 45.04 80) (end 45.04 87.96) (width 0.2) (layer "F.Cu") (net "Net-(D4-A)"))
 (segment (start 43.5 89.5) (end 43.5 93.42) (width 0.2) (layer "F.Cu") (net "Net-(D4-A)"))
 (segment (start 45.04 87.96) (end 43.5 89.5) (width 0.2) (layer "F.Cu") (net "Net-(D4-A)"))
 (segment (start 59.69 77.5) (end 45 77.5) (width 0.2) (layer "F.Cu") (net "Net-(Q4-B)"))
 (segment (start 45 77.5) (end 42.5 80) (width 0.2) (layer "F.Cu") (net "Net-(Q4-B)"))
 (segment (start 135.5 112.5) (end 135.5 104.58) (width 0.2) (layer "F.Cu") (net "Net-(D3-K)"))
 (segment (start 135.5 104.58) (end 131.92 101) (width 0.2) (layer "F.Cu") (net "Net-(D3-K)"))
 (segment (start 124.19 98.23) (end 138.42 84) (width 0.2) (layer "F.Cu") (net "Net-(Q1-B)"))
 (segment (start 124.19 109.5) (end 124.19 98.23) (width 0.2) (layer "F.Cu") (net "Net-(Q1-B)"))
 (segment (start 140.96 84) (end 140.96 99.88) (width 0.2) (layer "F.Cu") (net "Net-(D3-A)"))
 (segment (start 140.96 99.88) (end 142.08 101) (width 0.2) (layer "F.Cu") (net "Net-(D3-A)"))
 (segment (start 67.31 77.5) (end 122 77.5) (width 0.2) (layer "F.Cu") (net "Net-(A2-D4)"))
 (segment (start 122.905 89.5) (end 117.13 95.275) (width 0.2) (layer "F.Cu") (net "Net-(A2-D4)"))
 (segment (start 127.5 83) (end 127.5 89) (width 0.2) (layer "F.Cu") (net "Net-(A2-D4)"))
 (segment (start 127.5 89) (end 128 89.5) (width 0.2) (layer "F.Cu") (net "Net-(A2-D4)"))
 (segment (start 122 77.5) (end 127.5 83) (width 0.2) (layer "F.Cu") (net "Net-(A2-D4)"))
 (segment (start 128 89.5) (end 122.905 89.5) (width 0.2) (layer "F.Cu") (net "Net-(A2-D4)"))
 (segment (start 119.105 112.035) (end 124.19 117.12) (width 0.2) (layer "F.Cu") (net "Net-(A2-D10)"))
 (segment (start 117.13 112.035) (end 119.105 112.035) (width 0.2) (layer "F.Cu") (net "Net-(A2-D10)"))
 (segment (start 67.31 109.22) (end 67.31 106.995) (width 0.2) (layer "F.Cu") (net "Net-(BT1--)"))
 (segment (start 63.5 110.49) (end 64.77 109.22) (width 0.2) (layer "F.Cu") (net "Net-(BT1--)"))
 (segment (start 57.49 110.49) (end 63.5 110.49) (width 0.2) (layer "F.Cu") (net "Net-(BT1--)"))
 (segment (start 68.87 106.13) (end 68.87 105.435) (width 0.2) (layer "F.Cu") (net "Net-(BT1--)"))
 (segment (start 67.31 106.995) (end 68.87 105.435) (width 0.2) (layer "F.Cu") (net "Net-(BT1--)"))
 (segment (start 64.605 105.435) (end 68.87 105.435) (width 0.5) (layer "F.Cu") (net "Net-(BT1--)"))
 (segment (start 64.77 109.22) (end 65.085 109.22) (width 0.2) (layer "F.Cu") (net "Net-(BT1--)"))
 (segment (start 47.58 80) (end 56 80) (width 0.2) (layer "F.Cu") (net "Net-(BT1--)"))
 (segment (start 50.5 116.5) (end 60.03 116.5) (width 0.2) (layer "F.Cu") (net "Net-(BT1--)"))
 (segment (start 63 107.04) (end 64.605 105.435) (width 0.5) (layer "F.Cu") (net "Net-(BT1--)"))
 (segment (start 60.03 116.5) (end 67.31 109.22) (width 0.2) (layer "F.Cu") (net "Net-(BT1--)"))
 (segment (start 56 80) (end 56 109) (width 0.2) (layer "F.Cu") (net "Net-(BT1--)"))
 (segment (start 56 109) (end 57.49 110.49) (width 0.2) (layer "F.Cu") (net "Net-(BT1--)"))
 (segment (start 65.085 109.22) (end 67.31 106.995) (width 0.2) (layer "F.Cu") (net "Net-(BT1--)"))
 (segment (start 67.265 104.5) (end 68.87 102.895) (width 0.5) (layer "F.Cu") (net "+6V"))
 (segment (start 63 104.5) (end 67.265 104.5) (width 0.5) (layer "F.Cu") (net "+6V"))
 (segment (start 148.5 93) (end 148.5 119) (width 0.2) (layer "F.Cu") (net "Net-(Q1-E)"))
 (segment (start 143.695 122.195) (end 117.13 122.195) (width 0.2) (layer "F.Cu") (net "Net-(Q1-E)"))
 (segment (start 143.5 84) (end 143.5 88) (width 0.2) (layer "F.Cu") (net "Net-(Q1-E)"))
 (segment (start 148.5 119) (end 144.5 123) (width 0.2) (layer "F.Cu") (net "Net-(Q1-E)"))
 (segment (start 144.5 123) (end 143.695 122.195) (width 0.2) (layer "F.Cu") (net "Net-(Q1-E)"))
 (segment (start 128.345 122.195) (end 117.13 122.195) (width 0.2) (layer "F.Cu") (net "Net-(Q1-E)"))
 (segment (start 135.5 115.04) (end 128.345 122.195) (width 0.2) (layer "F.Cu") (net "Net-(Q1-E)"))
 (segment (start 143.5 88) (end 148.5 93) (width 0.2) (layer "F.Cu") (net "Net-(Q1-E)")))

